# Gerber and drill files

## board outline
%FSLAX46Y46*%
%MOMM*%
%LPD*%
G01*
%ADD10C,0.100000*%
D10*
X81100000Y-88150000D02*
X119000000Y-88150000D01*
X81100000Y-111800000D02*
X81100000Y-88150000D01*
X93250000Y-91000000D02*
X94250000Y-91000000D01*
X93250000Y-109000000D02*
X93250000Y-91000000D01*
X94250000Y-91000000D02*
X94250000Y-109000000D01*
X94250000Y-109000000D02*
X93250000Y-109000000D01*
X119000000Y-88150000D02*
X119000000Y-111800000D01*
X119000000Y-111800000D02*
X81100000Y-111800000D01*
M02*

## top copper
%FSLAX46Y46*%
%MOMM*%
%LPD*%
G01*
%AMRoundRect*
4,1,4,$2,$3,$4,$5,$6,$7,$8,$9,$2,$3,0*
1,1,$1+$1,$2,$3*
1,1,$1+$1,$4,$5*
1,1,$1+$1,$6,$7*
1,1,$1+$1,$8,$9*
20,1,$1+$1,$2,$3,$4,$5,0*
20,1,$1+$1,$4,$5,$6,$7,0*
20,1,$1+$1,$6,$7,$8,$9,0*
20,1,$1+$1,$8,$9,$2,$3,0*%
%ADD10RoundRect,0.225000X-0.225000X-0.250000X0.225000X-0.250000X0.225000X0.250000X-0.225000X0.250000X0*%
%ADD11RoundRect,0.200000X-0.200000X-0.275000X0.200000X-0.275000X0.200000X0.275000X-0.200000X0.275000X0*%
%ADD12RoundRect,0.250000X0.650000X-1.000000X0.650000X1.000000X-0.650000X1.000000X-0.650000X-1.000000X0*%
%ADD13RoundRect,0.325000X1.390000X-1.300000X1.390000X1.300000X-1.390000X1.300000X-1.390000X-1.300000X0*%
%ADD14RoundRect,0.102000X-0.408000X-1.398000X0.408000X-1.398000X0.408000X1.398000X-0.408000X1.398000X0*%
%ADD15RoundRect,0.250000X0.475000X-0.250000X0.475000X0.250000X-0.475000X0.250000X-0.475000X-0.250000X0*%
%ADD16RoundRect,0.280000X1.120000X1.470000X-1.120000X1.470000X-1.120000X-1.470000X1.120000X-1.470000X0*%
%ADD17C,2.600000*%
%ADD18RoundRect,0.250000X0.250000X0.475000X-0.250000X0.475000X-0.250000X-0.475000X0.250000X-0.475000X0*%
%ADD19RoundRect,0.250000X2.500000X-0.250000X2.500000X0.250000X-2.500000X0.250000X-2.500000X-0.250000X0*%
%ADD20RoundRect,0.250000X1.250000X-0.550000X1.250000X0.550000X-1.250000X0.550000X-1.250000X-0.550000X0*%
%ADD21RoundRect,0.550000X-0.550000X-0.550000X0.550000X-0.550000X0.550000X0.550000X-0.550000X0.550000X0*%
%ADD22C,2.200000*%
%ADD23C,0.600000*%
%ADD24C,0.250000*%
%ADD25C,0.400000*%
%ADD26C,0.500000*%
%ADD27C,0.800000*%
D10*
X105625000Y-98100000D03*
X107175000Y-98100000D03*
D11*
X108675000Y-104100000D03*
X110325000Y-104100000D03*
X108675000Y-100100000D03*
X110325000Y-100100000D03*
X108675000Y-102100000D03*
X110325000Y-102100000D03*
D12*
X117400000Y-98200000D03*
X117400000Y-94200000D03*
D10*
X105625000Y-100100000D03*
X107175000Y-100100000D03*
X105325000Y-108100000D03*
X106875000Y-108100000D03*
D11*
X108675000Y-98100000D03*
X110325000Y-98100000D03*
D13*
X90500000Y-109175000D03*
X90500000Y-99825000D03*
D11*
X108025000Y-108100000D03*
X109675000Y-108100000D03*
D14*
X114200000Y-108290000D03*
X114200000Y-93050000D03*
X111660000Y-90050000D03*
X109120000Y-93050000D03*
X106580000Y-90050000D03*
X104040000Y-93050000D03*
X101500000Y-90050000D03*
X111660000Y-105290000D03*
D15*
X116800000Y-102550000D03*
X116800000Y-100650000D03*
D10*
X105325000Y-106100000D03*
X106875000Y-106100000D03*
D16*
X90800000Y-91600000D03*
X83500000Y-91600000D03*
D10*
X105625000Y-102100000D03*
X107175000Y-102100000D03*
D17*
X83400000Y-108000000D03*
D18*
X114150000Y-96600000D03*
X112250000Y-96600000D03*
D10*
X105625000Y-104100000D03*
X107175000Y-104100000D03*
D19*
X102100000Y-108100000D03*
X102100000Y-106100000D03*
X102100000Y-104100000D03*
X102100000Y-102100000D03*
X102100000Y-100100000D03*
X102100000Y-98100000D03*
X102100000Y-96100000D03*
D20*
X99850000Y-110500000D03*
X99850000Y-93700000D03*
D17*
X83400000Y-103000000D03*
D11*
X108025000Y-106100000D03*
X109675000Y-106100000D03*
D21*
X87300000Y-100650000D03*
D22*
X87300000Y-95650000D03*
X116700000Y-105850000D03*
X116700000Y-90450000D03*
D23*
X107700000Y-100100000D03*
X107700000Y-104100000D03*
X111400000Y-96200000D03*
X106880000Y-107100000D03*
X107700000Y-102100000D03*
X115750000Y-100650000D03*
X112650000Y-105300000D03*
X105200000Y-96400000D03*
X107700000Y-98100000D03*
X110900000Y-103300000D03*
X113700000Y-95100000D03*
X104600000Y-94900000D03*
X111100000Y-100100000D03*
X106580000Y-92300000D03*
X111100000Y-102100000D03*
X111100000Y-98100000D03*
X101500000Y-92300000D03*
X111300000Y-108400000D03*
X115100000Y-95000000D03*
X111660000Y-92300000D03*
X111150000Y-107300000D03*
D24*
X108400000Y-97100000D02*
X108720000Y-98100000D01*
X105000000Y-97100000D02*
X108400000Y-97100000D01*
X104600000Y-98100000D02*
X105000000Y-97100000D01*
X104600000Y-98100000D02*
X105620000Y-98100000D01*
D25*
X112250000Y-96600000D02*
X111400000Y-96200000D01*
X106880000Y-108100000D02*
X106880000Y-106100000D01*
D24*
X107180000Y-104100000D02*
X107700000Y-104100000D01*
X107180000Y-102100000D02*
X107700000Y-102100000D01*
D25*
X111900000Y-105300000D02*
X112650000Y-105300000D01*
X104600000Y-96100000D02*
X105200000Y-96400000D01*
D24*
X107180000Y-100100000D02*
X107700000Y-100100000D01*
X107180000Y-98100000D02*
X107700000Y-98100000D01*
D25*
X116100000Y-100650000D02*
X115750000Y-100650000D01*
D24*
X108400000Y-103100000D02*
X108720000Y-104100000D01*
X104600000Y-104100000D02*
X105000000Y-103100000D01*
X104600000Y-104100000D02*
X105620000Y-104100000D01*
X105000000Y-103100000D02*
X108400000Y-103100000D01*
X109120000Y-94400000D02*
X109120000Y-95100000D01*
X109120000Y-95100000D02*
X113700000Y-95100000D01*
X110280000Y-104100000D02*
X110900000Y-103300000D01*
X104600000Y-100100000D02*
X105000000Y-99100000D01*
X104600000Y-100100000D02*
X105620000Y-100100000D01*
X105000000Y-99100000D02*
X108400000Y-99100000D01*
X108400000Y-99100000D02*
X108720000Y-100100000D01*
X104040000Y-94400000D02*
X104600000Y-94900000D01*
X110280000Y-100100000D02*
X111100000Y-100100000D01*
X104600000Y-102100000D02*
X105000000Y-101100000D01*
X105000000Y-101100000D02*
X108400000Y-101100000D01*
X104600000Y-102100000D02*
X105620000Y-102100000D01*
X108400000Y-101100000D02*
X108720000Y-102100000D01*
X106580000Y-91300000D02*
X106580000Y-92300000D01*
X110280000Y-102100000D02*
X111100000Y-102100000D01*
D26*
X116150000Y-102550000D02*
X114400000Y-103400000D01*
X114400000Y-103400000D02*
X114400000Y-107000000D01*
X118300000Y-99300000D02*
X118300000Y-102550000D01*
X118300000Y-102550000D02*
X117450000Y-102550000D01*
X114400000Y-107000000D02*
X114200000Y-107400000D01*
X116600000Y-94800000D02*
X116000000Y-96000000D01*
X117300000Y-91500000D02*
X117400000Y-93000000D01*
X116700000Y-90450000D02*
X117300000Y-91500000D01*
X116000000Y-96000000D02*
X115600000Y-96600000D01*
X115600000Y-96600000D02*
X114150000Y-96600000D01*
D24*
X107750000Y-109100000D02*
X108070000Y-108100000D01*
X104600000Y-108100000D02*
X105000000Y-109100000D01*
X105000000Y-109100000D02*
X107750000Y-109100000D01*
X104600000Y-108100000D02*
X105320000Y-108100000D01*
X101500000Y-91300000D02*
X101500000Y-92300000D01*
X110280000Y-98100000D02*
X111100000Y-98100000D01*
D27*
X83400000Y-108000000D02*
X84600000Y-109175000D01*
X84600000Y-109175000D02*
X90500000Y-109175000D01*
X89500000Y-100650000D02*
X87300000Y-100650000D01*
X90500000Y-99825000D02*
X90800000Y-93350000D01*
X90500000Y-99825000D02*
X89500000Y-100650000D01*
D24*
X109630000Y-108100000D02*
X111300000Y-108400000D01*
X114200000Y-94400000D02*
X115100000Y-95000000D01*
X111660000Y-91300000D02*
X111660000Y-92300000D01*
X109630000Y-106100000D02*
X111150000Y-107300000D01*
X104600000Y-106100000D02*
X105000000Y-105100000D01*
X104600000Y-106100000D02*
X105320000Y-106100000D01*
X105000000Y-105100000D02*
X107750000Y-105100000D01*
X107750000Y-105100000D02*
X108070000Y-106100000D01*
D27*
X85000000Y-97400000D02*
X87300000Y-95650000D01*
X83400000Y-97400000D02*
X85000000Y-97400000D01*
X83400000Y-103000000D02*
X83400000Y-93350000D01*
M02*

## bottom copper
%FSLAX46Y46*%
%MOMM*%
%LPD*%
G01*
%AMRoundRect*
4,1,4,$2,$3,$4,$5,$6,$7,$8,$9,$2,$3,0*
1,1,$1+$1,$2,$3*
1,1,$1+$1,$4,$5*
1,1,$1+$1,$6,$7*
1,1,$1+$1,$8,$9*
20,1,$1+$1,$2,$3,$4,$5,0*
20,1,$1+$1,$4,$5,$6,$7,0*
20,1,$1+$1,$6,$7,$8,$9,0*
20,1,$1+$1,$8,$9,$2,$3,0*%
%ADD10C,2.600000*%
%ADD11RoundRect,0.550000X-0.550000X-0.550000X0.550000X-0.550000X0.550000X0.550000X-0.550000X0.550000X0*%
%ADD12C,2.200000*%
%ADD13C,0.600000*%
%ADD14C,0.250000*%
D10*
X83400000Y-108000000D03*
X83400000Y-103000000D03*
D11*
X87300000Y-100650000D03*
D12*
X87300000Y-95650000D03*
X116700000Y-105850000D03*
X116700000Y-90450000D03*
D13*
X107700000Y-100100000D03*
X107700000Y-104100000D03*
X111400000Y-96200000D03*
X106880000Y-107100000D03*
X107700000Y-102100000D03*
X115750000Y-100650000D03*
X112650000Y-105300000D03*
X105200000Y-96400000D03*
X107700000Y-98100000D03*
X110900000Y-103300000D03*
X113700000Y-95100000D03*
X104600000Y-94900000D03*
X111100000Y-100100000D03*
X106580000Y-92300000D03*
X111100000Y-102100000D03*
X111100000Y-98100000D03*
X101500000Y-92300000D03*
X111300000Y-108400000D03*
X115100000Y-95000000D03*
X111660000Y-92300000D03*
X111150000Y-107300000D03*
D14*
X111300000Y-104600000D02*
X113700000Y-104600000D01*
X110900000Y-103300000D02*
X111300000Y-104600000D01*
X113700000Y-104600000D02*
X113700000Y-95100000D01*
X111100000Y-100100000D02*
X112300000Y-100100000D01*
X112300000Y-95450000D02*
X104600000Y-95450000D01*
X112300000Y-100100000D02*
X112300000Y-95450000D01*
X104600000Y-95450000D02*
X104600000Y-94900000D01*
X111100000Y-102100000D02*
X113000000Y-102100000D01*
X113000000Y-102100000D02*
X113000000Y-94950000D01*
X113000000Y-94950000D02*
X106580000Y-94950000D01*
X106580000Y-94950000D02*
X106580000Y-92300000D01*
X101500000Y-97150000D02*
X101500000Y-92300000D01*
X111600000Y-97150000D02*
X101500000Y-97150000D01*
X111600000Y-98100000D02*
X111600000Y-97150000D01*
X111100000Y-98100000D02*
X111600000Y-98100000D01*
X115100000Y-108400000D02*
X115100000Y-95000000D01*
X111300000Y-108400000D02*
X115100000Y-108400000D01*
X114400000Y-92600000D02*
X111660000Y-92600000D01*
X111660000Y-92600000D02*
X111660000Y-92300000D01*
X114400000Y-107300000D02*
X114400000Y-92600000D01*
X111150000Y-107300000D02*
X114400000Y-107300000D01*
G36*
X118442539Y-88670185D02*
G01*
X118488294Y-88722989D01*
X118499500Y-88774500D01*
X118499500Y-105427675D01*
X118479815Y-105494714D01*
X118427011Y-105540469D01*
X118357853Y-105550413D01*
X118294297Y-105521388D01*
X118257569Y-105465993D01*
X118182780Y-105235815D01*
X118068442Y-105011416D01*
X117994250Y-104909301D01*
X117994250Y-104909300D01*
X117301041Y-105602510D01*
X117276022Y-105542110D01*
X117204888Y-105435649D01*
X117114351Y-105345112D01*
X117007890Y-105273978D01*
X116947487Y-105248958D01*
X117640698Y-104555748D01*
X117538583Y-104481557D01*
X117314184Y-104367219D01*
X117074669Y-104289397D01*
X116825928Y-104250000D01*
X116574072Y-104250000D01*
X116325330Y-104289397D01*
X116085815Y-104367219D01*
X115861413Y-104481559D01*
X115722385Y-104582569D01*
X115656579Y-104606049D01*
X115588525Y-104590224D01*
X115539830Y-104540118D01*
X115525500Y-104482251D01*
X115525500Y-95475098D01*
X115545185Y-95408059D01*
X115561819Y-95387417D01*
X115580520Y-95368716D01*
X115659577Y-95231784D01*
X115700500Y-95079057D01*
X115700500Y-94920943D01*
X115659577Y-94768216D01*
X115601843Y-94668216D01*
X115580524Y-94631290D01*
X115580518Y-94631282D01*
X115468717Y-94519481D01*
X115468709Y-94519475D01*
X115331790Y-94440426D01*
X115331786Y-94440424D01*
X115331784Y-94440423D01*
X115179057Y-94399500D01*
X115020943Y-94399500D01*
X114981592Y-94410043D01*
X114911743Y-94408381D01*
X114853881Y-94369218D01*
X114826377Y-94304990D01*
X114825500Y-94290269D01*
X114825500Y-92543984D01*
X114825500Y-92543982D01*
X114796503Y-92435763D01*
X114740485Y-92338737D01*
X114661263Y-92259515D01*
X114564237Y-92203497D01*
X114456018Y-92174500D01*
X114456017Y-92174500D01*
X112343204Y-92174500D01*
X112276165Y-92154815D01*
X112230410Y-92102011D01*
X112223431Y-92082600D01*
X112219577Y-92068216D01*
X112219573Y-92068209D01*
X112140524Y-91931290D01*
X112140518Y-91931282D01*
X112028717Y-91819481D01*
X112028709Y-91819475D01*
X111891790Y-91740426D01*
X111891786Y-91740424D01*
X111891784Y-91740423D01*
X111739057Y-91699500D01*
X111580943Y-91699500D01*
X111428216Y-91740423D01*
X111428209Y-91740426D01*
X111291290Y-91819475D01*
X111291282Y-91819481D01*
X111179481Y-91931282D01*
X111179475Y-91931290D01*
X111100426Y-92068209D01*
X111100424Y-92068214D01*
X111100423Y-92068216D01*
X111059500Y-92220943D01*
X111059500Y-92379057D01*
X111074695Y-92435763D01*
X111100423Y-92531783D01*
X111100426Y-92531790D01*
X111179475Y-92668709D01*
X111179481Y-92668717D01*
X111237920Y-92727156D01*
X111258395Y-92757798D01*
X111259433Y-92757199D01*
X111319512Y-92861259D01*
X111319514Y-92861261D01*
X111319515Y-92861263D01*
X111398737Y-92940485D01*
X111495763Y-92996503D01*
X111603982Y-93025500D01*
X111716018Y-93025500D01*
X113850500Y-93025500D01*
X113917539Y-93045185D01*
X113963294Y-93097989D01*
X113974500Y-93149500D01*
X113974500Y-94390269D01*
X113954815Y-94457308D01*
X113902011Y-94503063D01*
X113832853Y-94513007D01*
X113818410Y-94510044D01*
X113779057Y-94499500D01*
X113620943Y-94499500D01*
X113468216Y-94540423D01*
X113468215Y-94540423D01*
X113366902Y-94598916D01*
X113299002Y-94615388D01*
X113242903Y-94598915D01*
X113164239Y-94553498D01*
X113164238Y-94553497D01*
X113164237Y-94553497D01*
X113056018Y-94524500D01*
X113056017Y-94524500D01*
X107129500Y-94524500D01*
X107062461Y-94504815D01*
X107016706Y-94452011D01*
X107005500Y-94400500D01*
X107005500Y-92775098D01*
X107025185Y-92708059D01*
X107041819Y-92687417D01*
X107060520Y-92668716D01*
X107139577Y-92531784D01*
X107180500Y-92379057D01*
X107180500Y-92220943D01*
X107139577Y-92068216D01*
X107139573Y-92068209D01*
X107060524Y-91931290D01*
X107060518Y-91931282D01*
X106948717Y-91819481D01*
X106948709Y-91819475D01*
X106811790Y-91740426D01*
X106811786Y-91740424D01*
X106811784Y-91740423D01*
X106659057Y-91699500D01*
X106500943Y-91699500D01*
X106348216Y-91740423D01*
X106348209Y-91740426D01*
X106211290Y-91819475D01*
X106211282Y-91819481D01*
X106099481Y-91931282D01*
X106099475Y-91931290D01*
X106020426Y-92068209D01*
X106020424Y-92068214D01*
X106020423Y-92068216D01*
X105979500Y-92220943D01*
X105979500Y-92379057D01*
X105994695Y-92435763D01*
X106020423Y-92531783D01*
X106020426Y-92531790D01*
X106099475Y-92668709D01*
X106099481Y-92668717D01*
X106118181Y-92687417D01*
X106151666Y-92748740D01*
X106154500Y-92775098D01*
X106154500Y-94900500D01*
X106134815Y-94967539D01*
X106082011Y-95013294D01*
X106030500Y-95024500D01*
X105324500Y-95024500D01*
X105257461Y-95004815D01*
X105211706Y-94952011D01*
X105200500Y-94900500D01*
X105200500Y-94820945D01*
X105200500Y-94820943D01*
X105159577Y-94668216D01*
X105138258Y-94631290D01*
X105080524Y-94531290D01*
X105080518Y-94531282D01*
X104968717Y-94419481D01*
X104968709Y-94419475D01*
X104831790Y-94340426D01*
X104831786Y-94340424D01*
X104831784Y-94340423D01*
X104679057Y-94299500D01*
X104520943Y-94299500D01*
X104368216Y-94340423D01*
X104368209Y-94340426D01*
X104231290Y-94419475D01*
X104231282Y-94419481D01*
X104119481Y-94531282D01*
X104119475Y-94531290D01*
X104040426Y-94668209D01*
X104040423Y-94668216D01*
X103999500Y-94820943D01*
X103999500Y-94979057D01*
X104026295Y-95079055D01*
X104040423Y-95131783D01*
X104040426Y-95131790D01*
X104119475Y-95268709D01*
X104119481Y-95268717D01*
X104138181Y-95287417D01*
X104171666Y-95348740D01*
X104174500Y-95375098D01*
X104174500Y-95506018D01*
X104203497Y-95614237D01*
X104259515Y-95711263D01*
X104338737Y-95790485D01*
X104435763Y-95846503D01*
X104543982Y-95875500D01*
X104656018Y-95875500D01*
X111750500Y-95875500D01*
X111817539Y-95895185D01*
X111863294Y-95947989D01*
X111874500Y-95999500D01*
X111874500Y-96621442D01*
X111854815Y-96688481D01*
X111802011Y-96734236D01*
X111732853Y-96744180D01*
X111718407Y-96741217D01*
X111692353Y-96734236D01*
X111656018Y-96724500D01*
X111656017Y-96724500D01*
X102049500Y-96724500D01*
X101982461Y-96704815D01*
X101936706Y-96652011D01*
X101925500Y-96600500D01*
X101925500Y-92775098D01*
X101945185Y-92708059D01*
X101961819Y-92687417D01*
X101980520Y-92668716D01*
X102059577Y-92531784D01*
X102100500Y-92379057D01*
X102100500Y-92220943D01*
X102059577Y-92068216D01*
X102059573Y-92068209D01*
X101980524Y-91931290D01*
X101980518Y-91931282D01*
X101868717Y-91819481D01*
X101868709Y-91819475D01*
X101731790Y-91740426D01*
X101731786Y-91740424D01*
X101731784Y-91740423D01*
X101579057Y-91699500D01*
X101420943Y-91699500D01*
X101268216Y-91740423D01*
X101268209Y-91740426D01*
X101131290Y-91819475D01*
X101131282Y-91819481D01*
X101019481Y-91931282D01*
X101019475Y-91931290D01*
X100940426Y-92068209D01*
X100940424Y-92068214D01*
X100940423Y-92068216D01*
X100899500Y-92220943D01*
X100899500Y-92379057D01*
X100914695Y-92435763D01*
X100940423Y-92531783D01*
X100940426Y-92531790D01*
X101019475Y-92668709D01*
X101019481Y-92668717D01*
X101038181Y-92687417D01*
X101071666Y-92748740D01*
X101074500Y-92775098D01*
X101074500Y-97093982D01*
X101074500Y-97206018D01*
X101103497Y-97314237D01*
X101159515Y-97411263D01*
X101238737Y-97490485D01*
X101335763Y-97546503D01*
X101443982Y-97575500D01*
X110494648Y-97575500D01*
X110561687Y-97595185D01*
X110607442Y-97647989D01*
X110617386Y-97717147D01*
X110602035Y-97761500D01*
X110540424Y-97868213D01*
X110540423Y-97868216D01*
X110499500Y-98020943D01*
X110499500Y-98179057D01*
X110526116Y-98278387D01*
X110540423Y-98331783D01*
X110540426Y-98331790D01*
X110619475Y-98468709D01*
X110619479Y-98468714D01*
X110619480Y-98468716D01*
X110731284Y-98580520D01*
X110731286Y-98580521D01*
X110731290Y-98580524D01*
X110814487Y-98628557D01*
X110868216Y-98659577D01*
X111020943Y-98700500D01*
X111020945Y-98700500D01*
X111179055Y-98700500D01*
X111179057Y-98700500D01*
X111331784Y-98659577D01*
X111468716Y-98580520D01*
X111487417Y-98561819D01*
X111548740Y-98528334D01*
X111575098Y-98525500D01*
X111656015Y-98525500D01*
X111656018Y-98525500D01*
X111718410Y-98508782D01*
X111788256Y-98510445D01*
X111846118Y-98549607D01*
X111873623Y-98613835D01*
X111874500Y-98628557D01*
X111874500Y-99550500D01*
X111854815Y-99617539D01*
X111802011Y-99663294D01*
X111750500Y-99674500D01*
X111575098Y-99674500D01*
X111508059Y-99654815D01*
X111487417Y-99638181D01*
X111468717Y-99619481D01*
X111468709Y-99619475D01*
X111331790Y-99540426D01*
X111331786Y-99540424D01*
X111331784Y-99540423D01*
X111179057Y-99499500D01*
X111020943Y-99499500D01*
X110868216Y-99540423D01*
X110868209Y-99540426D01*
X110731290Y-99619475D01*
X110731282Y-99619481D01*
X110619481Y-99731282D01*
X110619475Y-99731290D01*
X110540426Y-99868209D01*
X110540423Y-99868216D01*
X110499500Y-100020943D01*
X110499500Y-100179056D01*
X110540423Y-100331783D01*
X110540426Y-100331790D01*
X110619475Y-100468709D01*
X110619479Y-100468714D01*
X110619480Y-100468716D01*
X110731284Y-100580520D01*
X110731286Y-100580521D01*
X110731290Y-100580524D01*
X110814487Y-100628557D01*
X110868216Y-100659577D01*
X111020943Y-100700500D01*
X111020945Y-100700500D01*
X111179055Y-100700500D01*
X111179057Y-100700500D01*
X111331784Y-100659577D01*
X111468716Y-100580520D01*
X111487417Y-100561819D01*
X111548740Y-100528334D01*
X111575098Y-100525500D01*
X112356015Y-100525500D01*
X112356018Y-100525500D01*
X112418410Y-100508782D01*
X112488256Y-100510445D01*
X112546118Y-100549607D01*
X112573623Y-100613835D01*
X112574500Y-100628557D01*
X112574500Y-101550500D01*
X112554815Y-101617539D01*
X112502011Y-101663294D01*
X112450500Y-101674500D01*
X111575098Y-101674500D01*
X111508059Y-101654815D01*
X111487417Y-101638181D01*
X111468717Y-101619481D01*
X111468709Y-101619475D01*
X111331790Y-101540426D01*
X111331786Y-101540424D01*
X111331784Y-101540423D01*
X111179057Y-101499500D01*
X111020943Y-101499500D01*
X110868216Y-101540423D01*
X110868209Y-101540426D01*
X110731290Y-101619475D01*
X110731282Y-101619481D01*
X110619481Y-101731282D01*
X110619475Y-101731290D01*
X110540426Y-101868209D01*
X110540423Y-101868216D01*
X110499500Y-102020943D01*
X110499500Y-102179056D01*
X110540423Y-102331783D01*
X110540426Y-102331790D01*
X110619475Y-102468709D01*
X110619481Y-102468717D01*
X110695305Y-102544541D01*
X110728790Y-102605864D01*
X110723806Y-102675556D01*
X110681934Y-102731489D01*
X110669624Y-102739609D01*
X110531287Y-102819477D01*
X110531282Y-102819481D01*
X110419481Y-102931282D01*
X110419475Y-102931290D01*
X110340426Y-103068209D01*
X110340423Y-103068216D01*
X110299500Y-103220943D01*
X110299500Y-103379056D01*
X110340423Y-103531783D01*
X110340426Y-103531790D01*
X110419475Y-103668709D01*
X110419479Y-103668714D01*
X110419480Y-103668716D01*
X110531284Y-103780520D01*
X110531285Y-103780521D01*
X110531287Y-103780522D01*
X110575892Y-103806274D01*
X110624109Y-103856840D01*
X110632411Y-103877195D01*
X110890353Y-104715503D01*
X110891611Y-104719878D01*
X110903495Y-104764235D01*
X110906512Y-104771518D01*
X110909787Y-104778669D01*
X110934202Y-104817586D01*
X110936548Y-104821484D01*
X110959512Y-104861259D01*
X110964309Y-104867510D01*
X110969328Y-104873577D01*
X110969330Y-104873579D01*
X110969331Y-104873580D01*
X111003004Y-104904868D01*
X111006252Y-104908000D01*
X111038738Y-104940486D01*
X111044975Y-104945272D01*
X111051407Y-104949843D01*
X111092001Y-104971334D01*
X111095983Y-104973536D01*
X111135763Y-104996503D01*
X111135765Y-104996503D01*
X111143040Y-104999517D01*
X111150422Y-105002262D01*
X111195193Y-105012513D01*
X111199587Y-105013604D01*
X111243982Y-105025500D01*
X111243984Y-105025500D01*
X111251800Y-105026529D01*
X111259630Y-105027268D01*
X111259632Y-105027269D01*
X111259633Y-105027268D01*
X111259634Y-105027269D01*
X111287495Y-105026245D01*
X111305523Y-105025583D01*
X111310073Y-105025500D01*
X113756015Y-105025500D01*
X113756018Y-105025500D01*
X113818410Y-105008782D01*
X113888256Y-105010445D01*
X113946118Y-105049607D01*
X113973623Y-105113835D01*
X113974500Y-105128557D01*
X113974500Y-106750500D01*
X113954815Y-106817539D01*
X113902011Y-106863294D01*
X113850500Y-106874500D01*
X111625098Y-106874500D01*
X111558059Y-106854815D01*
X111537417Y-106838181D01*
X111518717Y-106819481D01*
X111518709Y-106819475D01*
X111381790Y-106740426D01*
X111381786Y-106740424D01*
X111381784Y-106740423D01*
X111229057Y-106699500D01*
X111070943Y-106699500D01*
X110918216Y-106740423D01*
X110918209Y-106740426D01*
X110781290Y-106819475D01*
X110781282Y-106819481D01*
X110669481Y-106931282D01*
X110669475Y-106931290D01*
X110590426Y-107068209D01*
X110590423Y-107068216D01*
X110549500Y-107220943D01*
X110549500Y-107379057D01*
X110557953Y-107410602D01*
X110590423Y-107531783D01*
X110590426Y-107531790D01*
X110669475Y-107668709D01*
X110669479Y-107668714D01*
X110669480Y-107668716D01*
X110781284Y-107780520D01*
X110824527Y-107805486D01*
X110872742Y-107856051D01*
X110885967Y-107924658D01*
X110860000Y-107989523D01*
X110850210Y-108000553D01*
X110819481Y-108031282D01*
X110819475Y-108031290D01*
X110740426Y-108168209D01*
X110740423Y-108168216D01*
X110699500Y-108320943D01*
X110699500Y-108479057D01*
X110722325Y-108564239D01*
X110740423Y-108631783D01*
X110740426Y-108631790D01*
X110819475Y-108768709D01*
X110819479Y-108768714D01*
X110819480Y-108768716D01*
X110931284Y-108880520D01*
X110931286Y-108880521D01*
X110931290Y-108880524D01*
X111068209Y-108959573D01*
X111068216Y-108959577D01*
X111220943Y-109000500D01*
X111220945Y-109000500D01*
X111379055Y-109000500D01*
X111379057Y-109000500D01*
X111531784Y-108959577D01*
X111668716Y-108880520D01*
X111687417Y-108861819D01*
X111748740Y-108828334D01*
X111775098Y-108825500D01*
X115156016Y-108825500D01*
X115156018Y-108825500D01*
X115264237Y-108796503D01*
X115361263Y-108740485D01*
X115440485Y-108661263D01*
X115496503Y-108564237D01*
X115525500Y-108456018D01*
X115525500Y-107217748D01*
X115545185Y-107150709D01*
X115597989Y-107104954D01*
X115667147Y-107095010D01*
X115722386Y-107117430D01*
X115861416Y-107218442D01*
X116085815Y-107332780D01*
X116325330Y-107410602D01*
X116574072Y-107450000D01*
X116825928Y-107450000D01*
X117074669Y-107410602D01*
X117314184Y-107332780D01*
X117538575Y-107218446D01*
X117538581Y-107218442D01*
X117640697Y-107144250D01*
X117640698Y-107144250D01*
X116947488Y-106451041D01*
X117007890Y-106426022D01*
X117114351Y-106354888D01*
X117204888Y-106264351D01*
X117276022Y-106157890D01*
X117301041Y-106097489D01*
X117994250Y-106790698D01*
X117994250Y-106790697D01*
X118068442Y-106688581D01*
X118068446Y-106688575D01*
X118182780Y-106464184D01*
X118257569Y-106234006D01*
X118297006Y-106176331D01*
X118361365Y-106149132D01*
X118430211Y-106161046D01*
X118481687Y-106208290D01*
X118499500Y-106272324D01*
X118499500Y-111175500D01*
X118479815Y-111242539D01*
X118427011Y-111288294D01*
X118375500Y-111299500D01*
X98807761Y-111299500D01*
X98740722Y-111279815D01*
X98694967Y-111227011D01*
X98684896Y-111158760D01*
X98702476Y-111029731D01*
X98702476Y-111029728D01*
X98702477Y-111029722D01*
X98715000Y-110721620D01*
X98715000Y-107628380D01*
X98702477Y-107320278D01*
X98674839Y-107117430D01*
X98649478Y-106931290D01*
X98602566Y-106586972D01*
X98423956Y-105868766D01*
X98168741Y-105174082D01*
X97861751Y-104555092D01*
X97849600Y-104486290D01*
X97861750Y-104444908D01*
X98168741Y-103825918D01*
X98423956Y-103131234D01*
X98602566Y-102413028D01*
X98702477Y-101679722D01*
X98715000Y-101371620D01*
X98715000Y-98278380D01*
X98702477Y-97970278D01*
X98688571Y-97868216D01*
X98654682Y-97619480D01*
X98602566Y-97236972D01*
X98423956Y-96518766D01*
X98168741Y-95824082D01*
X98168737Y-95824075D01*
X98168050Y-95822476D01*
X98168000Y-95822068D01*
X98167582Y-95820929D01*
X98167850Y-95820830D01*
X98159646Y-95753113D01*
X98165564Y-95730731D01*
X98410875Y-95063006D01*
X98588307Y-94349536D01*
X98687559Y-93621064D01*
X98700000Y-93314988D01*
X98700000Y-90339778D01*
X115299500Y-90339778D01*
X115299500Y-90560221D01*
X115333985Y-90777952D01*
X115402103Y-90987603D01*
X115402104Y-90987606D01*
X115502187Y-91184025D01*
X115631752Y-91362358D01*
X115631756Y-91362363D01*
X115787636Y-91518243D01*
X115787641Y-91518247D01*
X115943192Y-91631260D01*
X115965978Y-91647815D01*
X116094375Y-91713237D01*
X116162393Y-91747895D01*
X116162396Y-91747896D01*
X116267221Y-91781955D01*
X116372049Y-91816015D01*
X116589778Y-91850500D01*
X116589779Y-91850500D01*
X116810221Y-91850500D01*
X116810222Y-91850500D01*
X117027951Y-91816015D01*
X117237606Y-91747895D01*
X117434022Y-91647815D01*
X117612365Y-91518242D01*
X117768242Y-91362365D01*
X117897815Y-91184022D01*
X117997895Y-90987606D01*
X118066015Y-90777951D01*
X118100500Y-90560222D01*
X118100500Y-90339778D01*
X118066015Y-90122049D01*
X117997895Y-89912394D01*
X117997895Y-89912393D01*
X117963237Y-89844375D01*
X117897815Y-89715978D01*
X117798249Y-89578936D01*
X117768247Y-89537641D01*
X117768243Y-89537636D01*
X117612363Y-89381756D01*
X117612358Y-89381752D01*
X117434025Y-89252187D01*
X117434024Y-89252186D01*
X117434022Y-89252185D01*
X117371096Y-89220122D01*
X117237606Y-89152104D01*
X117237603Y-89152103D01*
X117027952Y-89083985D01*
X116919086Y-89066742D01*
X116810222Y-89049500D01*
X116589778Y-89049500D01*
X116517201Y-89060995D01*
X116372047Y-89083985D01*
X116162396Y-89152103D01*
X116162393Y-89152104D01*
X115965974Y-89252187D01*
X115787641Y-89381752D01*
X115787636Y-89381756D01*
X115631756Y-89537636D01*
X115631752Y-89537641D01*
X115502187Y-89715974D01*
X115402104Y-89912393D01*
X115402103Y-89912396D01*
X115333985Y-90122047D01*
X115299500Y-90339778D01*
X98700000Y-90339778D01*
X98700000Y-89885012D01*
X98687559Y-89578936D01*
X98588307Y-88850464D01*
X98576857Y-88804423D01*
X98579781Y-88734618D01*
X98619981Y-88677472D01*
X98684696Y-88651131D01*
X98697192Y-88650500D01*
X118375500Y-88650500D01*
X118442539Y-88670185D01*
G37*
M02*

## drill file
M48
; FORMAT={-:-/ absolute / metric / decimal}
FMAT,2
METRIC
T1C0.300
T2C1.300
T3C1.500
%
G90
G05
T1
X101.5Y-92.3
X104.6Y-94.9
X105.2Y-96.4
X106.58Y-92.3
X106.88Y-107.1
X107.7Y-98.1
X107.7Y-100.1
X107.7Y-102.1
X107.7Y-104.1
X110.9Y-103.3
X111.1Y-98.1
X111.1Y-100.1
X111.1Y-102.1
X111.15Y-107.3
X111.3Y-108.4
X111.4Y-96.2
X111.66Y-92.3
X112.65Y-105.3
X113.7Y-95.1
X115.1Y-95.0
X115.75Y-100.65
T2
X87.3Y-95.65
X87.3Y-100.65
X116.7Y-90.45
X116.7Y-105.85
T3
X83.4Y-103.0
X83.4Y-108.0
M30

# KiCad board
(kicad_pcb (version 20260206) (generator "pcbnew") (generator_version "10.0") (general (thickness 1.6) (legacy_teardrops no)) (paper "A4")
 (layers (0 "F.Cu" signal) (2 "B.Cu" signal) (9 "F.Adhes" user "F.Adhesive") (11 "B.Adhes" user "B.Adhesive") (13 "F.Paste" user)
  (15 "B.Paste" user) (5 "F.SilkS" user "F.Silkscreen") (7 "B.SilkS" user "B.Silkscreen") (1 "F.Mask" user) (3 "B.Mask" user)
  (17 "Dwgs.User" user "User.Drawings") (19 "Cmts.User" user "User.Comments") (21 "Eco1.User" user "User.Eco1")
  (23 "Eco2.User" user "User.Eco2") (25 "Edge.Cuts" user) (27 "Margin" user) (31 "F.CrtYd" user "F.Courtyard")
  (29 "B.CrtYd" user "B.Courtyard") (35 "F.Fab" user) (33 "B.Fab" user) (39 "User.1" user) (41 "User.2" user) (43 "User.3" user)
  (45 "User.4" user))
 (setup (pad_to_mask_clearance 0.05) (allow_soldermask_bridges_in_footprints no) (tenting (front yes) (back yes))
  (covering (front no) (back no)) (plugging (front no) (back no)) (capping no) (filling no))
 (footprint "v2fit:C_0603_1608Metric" (layer "F.Cu") (at 106.4 98.1)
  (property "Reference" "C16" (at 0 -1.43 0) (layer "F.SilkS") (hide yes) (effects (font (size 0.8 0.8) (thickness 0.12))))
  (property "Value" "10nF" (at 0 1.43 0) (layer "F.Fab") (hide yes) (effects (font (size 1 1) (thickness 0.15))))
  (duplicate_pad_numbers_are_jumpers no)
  (pad "1" smd roundrect (at -0.775 0) (size 0.9 0.95) (layers "F.Cu" "F.Mask" "F.Paste") (roundrect_rratio 0.25) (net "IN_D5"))
  (pad "2" smd roundrect (at 0.775 0) (size 0.9 0.95) (layers "F.Cu" "F.Mask" "F.Paste") (roundrect_rratio 0.25) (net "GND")))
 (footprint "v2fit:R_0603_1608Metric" (layer "F.Cu") (at 109.5 104.1)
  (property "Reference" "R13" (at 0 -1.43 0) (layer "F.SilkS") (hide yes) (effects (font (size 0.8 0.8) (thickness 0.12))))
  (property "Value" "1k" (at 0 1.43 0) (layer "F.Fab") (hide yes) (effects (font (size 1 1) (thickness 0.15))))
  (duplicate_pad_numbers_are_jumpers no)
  (pad "1" smd roundrect (at -0.825 0) (size 0.8 0.95) (layers "F.Cu" "F.Mask" "F.Paste") (roundrect_rratio 0.25) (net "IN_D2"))
  (pad "2" smd roundrect (at 0.825 0) (size 0.8 0.95) (layers "F.Cu" "F.Mask" "F.Paste") (roundrect_rratio 0.25) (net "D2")))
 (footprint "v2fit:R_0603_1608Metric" (layer "F.Cu") (at 109.5 100.1)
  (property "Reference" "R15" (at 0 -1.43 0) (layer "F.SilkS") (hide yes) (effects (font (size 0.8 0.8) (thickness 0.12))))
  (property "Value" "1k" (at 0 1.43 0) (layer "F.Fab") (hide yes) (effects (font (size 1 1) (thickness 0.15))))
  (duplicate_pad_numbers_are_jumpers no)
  (pad "1" smd roundrect (at -0.825 0) (size 0.8 0.95) (layers "F.Cu" "F.Mask" "F.Paste") (roundrect_rratio 0.25) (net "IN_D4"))
  (pad "2" smd roundrect (at 0.825 0) (size 0.8 0.95) (layers "F.Cu" "F.Mask" "F.Paste") (roundrect_rratio 0.25) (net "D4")))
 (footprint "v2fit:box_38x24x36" (layer "F.Cu") (at 100 100)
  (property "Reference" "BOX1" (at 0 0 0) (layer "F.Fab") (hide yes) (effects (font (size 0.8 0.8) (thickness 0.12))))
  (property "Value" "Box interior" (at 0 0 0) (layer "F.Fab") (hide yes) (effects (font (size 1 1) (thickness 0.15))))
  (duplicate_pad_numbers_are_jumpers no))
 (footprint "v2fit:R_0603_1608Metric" (layer "F.Cu") (at 109.5 102.1)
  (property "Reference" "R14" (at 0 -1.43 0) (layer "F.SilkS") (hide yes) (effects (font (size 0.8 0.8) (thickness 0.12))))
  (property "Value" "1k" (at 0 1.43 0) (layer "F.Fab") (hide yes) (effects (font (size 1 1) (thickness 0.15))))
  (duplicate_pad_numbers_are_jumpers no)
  (pad "1" smd roundrect (at -0.825 0) (size 0.8 0.95) (layers "F.Cu" "F.Mask" "F.Paste") (roundrect_rratio 0.25) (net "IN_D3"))
  (pad "2" smd roundrect (at 0.825 0) (size 0.8 0.95) (layers "F.Cu" "F.Mask" "F.Paste") (roundrect_rratio 0.25) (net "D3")))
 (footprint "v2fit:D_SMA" (layer "F.Cu") (at 117.4 96.2 90)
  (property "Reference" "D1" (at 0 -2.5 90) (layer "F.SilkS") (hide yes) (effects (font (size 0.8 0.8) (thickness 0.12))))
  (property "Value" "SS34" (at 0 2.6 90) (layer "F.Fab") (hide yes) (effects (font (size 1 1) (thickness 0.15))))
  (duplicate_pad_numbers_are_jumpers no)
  (pad "1" smd roundrect (at -2 0 90) (size 2.5 1.8) (layers "F.Cu" "F.Mask" "F.Paste") (roundrect_rratio 0.1388888889) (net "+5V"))
  (pad "2" smd roundrect (at 2 0 90) (size 2.5 1.8) (layers "F.Cu" "F.Mask" "F.Paste") (roundrect_rratio 0.1388888889) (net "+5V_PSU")))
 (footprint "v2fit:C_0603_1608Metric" (layer "F.Cu") (at 106.4 100.1)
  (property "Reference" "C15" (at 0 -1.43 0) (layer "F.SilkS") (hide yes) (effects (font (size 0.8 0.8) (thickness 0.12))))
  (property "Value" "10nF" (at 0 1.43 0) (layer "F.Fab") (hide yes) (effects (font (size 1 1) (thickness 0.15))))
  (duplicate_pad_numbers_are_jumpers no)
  (pad "1" smd roundrect (at -0.775 0) (size 0.9 0.95) (layers "F.Cu" "F.Mask" "F.Paste") (roundrect_rratio 0.25) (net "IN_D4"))
  (pad "2" smd roundrect (at 0.775 0) (size 0.9 0.95) (layers "F.Cu" "F.Mask" "F.Paste") (roundrect_rratio 0.25) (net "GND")))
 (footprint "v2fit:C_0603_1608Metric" (layer "F.Cu") (at 106.1 108.1)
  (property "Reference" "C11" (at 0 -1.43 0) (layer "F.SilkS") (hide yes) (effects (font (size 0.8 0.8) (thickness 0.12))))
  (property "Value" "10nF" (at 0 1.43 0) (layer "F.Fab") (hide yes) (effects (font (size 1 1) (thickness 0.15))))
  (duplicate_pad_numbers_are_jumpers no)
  (pad "1" smd roundrect (at -0.775 0) (size 0.9 0.95) (layers "F.Cu" "F.Mask" "F.Paste") (roundrect_rratio 0.25) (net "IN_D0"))
  (pad "2" smd roundrect (at 0.775 0) (size 0.9 0.95) (layers "F.Cu" "F.Mask" "F.Paste") (roundrect_rratio 0.25) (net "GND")))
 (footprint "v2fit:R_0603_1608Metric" (layer "F.Cu") (at 109.5 98.1)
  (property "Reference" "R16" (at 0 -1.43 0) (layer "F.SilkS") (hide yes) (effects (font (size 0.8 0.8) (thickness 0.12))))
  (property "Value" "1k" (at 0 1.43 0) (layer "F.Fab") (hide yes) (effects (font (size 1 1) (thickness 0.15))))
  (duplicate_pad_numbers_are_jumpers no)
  (pad "1" smd roundrect (at -0.825 0) (size 0.8 0.95) (layers "F.Cu" "F.Mask" "F.Paste") (roundrect_rratio 0.25) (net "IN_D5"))
  (pad "2" smd roundrect (at 0.825 0) (size 0.8 0.95) (layers "F.Cu" "F.Mask" "F.Paste") (roundrect_rratio 0.25) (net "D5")))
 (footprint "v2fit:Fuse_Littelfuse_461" (layer "F.Cu") (at 90.5 104.5 90)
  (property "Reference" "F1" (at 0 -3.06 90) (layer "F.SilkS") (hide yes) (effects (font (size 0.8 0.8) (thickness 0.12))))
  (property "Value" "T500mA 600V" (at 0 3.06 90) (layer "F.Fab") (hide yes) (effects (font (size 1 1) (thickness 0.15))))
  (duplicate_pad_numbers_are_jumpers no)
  (pad "1" smd roundrect (at -4.675 0 90) (size 3.25 3.43) (layers "F.Cu" "F.Mask" "F.Paste") (roundrect_rratio 0.1) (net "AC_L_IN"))
  (pad "2" smd roundrect (at 4.675 0 90) (size 3.25 3.43) (layers "F.Cu" "F.Mask" "F.Paste") (roundrect_rratio 0.1) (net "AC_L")))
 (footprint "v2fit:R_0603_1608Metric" (layer "F.Cu") (at 108.85 108.1)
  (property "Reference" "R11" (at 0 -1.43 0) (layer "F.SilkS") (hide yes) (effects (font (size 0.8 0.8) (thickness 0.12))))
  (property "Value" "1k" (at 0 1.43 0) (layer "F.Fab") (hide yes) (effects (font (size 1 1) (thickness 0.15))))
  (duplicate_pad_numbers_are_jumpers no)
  (pad "1" smd roundrect (at -0.825 0) (size 0.8 0.95) (layers "F.Cu" "F.Mask" "F.Paste") (roundrect_rratio 0.25) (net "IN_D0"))
  (pad "2" smd roundrect (at 0.825 0) (size 0.8 0.95) (layers "F.Cu" "F.Mask" "F.Paste") (roundrect_rratio 0.25) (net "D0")))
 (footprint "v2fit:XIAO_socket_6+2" (layer "F.Cu") (at 106.58 99.17)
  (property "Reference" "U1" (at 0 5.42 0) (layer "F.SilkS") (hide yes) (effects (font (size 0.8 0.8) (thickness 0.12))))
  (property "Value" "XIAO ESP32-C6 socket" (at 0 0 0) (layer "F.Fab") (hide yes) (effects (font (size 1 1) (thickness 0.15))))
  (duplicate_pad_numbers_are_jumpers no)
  (pad "5V" smd roundrect (at 7.62 9.12) (size 1.02 3) (layers "F.Cu" "F.Mask" "F.Paste") (roundrect_rratio 0.1) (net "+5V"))
  (pad "D0" smd roundrect (at 7.62 -6.12) (size 1.02 3) (layers "F.Cu" "F.Mask" "F.Paste") (roundrect_rratio 0.1) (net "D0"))
  (pad "D1" smd roundrect (at 5.08 -9.12) (size 1.02 3) (layers "F.Cu" "F.Mask" "F.Paste") (roundrect_rratio 0.1) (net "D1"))
  (pad "D2" smd roundrect (at 2.54 -6.12) (size 1.02 3) (layers "F.Cu" "F.Mask" "F.Paste") (roundrect_rratio 0.1) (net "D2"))
  (pad "D3" smd roundrect (at 0 -9.12) (size 1.02 3) (layers "F.Cu" "F.Mask" "F.Paste") (roundrect_rratio 0.1) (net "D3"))
  (pad "D4" smd roundrect (at -2.54 -6.12) (size 1.02 3) (layers "F.Cu" "F.Mask" "F.Paste") (roundrect_rratio 0.1) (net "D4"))
  (pad "D5" smd roundrect (at -5.08 -9.12) (size 1.02 3) (layers "F.Cu" "F.Mask" "F.Paste") (roundrect_rratio 0.1) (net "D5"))
  (pad "GND" smd roundrect (at 5.08 6.12) (size 1.02 3) (layers "F.Cu" "F.Mask" "F.Paste") (roundrect_rratio 0.1) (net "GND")))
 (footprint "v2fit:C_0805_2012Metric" (layer "F.Cu") (at 116.8 101.6 90)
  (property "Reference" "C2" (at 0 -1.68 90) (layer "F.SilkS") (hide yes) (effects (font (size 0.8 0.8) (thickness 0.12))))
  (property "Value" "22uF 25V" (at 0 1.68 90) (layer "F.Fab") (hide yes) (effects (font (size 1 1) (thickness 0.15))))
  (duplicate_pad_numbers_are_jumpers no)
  (pad "1" smd roundrect (at -0.95 0 90) (size 1 1.45) (layers "F.Cu" "F.Mask" "F.Paste") (roundrect_rratio 0.25) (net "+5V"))
  (pad "2" smd roundrect (at 0.95 0 90) (size 1 1.45) (layers "F.Cu" "F.Mask" "F.Paste") (roundrect_rratio 0.25) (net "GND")))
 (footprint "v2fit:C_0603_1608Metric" (layer "F.Cu") (at 106.1 106.1)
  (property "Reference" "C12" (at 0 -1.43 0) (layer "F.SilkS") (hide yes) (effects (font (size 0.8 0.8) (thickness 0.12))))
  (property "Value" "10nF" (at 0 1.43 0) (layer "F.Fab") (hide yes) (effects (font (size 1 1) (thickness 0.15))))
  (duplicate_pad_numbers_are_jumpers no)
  (pad "1" smd roundrect (at -0.775 0) (size 0.9 0.95) (layers "F.Cu" "F.Mask" "F.Paste") (roundrect_rratio 0.25) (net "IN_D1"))
  (pad "2" smd roundrect (at 0.775 0) (size 0.9 0.95) (layers "F.Cu" "F.Mask" "F.Paste") (roundrect_rratio 0.25) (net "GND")))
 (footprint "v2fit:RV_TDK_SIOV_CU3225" (layer "F.Cu") (at 87.15 91.6 180)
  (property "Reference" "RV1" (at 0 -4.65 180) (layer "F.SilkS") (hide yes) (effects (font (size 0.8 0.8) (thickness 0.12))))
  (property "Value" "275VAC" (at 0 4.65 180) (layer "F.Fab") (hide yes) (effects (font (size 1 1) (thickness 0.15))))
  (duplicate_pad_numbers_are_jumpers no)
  (pad "1" smd roundrect (at -3.65 0 180) (size 2.8 3.5) (layers "F.Cu" "F.Mask" "F.Paste") (roundrect_rratio 0.1) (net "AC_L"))
  (pad "2" smd roundrect (at 3.65 0 180) (size 2.8 3.5) (layers "F.Cu" "F.Mask" "F.Paste") (roundrect_rratio 0.1) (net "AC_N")))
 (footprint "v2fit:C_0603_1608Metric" (layer "F.Cu") (at 106.4 102.1)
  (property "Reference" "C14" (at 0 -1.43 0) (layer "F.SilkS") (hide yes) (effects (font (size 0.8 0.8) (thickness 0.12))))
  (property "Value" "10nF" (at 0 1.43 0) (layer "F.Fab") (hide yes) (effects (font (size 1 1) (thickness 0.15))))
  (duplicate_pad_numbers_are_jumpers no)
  (pad "1" smd roundrect (at -0.775 0) (size 0.9 0.95) (layers "F.Cu" "F.Mask" "F.Paste") (roundrect_rratio 0.25) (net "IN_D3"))
  (pad "2" smd roundrect (at 0.775 0) (size 0.9 0.95) (layers "F.Cu" "F.Mask" "F.Paste") (roundrect_rratio 0.25) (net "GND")))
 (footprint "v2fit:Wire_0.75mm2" (layer "F.Cu") (at 83.4 108)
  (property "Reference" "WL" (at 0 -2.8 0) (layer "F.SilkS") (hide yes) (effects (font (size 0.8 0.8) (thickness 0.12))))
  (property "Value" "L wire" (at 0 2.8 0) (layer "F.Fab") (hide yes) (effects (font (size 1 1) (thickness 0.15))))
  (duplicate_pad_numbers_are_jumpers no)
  (pad "1" thru_hole circle (at 0 0) (size 2.6 2.6) (drill 1.5) (layers "*.Cu" "*.Mask") (remove_unused_layers no) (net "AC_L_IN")))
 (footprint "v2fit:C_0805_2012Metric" (layer "F.Cu") (at 113.2 96.6 180)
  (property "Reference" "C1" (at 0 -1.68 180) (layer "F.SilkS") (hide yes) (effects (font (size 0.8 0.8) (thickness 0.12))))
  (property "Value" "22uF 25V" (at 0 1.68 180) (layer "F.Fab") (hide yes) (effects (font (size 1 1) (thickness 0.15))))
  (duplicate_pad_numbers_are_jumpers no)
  (pad "1" smd roundrect (at -0.95 0 180) (size 1 1.45) (layers "F.Cu" "F.Mask" "F.Paste") (roundrect_rratio 0.25) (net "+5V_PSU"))
  (pad "2" smd roundrect (at 0.95 0 180) (size 1 1.45) (layers "F.Cu" "F.Mask" "F.Paste") (roundrect_rratio 0.25) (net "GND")))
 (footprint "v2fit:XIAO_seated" (layer "F.Cu") (at 106.58 99.17)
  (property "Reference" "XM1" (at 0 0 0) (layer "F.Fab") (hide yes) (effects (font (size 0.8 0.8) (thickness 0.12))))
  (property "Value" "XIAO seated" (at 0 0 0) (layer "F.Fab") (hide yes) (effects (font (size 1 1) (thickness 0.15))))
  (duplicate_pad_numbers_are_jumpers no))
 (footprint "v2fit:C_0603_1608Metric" (layer "F.Cu") (at 106.4 104.1)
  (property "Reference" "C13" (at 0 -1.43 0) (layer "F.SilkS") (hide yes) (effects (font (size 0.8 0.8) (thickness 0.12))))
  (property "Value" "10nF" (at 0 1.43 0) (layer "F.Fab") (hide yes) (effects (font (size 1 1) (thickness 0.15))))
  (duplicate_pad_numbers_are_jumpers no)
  (pad "1" smd roundrect (at -0.775 0) (size 0.9 0.95) (layers "F.Cu" "F.Mask" "F.Paste") (roundrect_rratio 0.25) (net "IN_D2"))
  (pad "2" smd roundrect (at 0.775 0) (size 0.9 0.95) (layers "F.Cu" "F.Mask" "F.Paste") (roundrect_rratio 0.25) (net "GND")))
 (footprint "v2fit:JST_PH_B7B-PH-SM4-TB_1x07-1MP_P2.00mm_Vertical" (layer "F.Cu") (at 101.6 102.1 90)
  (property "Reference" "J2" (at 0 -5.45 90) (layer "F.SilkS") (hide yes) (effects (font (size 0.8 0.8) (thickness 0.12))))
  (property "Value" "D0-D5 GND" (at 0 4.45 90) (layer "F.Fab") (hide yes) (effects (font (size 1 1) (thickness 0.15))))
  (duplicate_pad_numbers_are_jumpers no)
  (pad "1" smd roundrect (at -6 0.5 90) (size 1 5.5) (layers "F.Cu" "F.Mask" "F.Paste") (roundrect_rratio 0.25) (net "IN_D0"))
  (pad "2" smd roundrect (at -4 0.5 90) (size 1 5.5) (layers "F.Cu" "F.Mask" "F.Paste") (roundrect_rratio 0.25) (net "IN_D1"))
  (pad "3" smd roundrect (at -2 0.5 90) (size 1 5.5) (layers "F.Cu" "F.Mask" "F.Paste") (roundrect_rratio 0.25) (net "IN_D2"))
  (pad "4" smd roundrect (at 0 0.5 90) (size 1 5.5) (layers "F.Cu" "F.Mask" "F.Paste") (roundrect_rratio 0.25) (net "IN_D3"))
  (pad "5" smd roundrect (at 2 0.5 90) (size 1 5.5) (layers "F.Cu" "F.Mask" "F.Paste") (roundrect_rratio 0.25) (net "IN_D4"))
  (pad "6" smd roundrect (at 4 0.5 90) (size 1 5.5) (layers "F.Cu" "F.Mask" "F.Paste") (roundrect_rratio 0.25) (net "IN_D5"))
  (pad "7" smd roundrect (at 6 0.5 90) (size 1 5.5) (layers "F.Cu" "F.Mask" "F.Paste") (roundrect_rratio 0.25) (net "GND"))
  (pad "MP" smd roundrect (at -8.4 -1.75 90) (size 1.6 3) (layers "F.Cu" "F.Mask" "F.Paste") (roundrect_rratio 0.15625))
  (pad "MP" smd roundrect (at 8.4 -1.75 90) (size 1.6 3) (layers "F.Cu" "F.Mask" "F.Paste") (roundrect_rratio 0.15625)))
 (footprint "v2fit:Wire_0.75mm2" (layer "F.Cu") (at 83.4 103)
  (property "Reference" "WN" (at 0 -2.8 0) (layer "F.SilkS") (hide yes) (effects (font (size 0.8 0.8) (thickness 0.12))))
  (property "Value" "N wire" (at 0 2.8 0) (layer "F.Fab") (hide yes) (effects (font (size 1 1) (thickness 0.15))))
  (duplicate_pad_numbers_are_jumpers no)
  (pad "1" thru_hole circle (at 0 0) (size 2.6 2.6) (drill 1.5) (layers "*.Cu" "*.Mask") (remove_unused_layers no) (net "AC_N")))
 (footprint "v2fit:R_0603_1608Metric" (layer "F.Cu") (at 108.85 106.1)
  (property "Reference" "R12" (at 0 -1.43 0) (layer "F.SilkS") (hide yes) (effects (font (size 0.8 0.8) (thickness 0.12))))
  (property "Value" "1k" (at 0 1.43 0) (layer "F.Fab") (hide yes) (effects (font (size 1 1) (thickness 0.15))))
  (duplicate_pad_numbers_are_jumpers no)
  (pad "1" smd roundrect (at -0.825 0) (size 0.8 0.95) (layers "F.Cu" "F.Mask" "F.Paste") (roundrect_rratio 0.25) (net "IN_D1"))
  (pad "2" smd roundrect (at 0.825 0) (size 0.8 0.95) (layers "F.Cu" "F.Mask" "F.Paste") (roundrect_rratio 0.25) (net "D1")))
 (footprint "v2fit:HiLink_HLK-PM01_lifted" (layer "B.Cu") (at 87.3 100.65)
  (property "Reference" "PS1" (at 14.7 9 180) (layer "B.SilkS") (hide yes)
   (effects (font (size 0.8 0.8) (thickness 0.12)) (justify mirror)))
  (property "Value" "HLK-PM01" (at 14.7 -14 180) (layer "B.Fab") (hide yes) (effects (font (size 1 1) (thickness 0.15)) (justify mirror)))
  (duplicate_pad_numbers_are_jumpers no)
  (pad "1" thru_hole roundrect (at 0 0) (size 2.2 2.2) (drill 1.3) (layers "*.Cu" "*.Mask") (remove_unused_layers no)
   (roundrect_rratio 0.25) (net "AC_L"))
  (pad "2" thru_hole circle (at 0 -5) (size 2.2 2.2) (drill 1.3) (layers "*.Cu" "*.Mask") (remove_unused_layers no) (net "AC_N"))
  (pad "3" thru_hole circle (at 29.4 5.2) (size 2.2 2.2) (drill 1.3) (layers "*.Cu" "*.Mask") (remove_unused_layers no) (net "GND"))
  (pad "4" thru_hole circle (at 29.4 -10.2) (size 2.2 2.2) (drill 1.3) (layers "*.Cu" "*.Mask") (remove_unused_layers no) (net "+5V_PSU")))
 (gr_line (start 81.1 88.15) (end 119 88.15) (stroke (width 0.1) (type default)) (layer "Edge.Cuts"))
 (gr_line (start 81.1 111.8) (end 81.1 88.15) (stroke (width 0.1) (type default)) (layer "Edge.Cuts"))
 (gr_line (start 93.25 91) (end 94.25 91) (stroke (width 0.1) (type default)) (layer "Edge.Cuts"))
 (gr_line (start 93.25 109) (end 93.25 91) (stroke (width 0.1) (type default)) (layer "Edge.Cuts"))
 (gr_line (start 94.25 91) (end 94.25 109) (stroke (width 0.1) (type default)) (layer "Edge.Cuts"))
 (gr_line (start 94.25 109) (end 93.25 109) (stroke (width 0.1) (type default)) (layer "Edge.Cuts"))
 (gr_line (start 119 88.15) (end 119 111.8) (stroke (width 0.1) (type default)) (layer "Edge.Cuts"))
 (gr_line (start 119 111.8) (end 81.1 111.8) (stroke (width 0.1) (type default)) (layer "Edge.Cuts"))
 (segment (start 108.4 97.1) (end 108.72 98.1) (width 0.25) (layer "F.Cu") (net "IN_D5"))
 (segment (start 105 97.1) (end 108.4 97.1) (width 0.25) (layer "F.Cu") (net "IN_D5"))
 (segment (start 104.6 98.1) (end 105 97.1) (width 0.25) (layer "F.Cu") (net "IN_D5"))
 (segment (start 104.6 98.1) (end 105.62 98.1) (width 0.25) (layer "F.Cu") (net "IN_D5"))
 (segment (start 112.25 96.6) (end 111.4 96.2) (width 0.4) (layer "F.Cu") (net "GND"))
 (segment (start 106.88 108.1) (end 106.88 106.1) (width 0.4) (layer "F.Cu") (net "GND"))
 (segment (start 107.18 104.1) (end 107.7 104.1) (width 0.25) (layer "F.Cu") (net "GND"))
 (segment (start 107.18 102.1) (end 107.7 102.1) (width 0.25) (layer "F.Cu") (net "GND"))
 (segment (start 111.9 105.3) (end 112.65 105.3) (width 0.4) (layer "F.Cu") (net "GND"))
 (segment (start 104.6 96.1) (end 105.2 96.4) (width 0.4) (layer "F.Cu") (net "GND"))
 (segment (start 107.18 100.1) (end 107.7 100.1) (width 0.25) (layer "F.Cu") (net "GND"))
 (segment (start 107.18 98.1) (end 107.7 98.1) (width 0.25) (layer "F.Cu") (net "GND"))
 (segment (start 116.1 100.65) (end 115.75 100.65) (width 0.4) (layer "F.Cu") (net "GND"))
 (via (at 107.7 100.1) (size 0.6) (drill 0.3) (layers "F.Cu" "B.Cu") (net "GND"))
 (via (at 107.7 104.1) (size 0.6) (drill 0.3) (layers "F.Cu" "B.Cu") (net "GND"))
 (via (at 111.4 96.2) (size 0.6) (drill 0.3) (layers "F.Cu" "B.Cu") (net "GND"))
 (via (at 106.88 107.1) (size 0.6) (drill 0.3) (layers "F.Cu" "B.Cu") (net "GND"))
 (via (at 107.7 102.1) (size 0.6) (drill 0.3) (layers "F.Cu" "B.Cu") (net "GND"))
 (via (at 115.75 100.65) (size 0.6) (drill 0.3) (layers "F.Cu" "B.Cu") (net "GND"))
 (via (at 112.65 105.3) (size 0.6) (drill 0.3) (layers "F.Cu" "B.Cu") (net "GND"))
 (via (at 105.2 96.4) (size 0.6) (drill 0.3) (layers "F.Cu" "B.Cu") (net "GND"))
 (via (at 107.7 98.1) (size 0.6) (drill 0.3) (layers "F.Cu" "B.Cu") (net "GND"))
 (segment (start 108.4 103.1) (end 108.72 104.1) (width 0.25) (layer "F.Cu") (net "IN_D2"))
 (segment (start 104.6 104.1) (end 105 103.1) (width 0.25) (layer "F.Cu") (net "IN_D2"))
 (segment (start 104.6 104.1) (end 105.62 104.1) (width 0.25) (layer "F.Cu") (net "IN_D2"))
 (segment (start 105 103.1) (end 108.4 103.1) (width 0.25) (layer "F.Cu") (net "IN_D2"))
 (segment (start 109.12 94.4) (end 109.12 95.1) (width 0.25) (layer "F.Cu") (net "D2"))
 (segment (start 109.12 95.1) (end 113.7 95.1) (width 0.25) (layer "F.Cu") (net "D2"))
 (segment (start 110.28 104.1) (end 110.9 103.3) (width 0.25) (layer "F.Cu") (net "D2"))
 (via (at 110.9 103.3) (size 0.6) (drill 0.3) (layers "F.Cu" "B.Cu") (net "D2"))
 (via (at 113.7 95.1) (size 0.6) (drill 0.3) (layers "F.Cu" "B.Cu") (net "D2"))
 (segment (start 111.3 104.6) (end 113.7 104.6) (width 0.25) (layer "B.Cu") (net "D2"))
 (segment (start 110.9 103.3) (end 111.3 104.6) (width 0.25) (layer "B.Cu") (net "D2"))
 (segment (start 113.7 104.6) (end 113.7 95.1) (width 0.25) (layer "B.Cu") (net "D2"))
 (segment (start 104.6 100.1) (end 105 99.1) (width 0.25) (layer "F.Cu") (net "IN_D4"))
 (segment (start 104.6 100.1) (end 105.62 100.1) (width 0.25) (layer "F.Cu") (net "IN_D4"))
 (segment (start 105 99.1) (end 108.4 99.1) (width 0.25) (layer "F.Cu") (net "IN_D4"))
 (segment (start 108.4 99.1) (end 108.72 100.1) (width 0.25) (layer "F.Cu") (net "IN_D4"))
 (segment (start 104.04 94.4) (end 104.6 94.9) (width 0.25) (layer "F.Cu") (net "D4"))
 (segment (start 110.28 100.1) (end 111.1 100.1) (width 0.25) (layer "F.Cu") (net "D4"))
 (via (at 104.6 94.9) (size 0.6) (drill 0.3) (layers "F.Cu" "B.Cu") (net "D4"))
 (via (at 111.1 100.1) (size 0.6) (drill 0.3) (layers "F.Cu" "B.Cu") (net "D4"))
 (segment (start 111.1 100.1) (end 112.3 100.1) (width 0.25) (layer "B.Cu") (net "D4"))
 (segment (start 112.3 95.45) (end 104.6 95.45) (width 0.25) (layer "B.Cu") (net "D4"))
 (segment (start 112.3 100.1) (end 112.3 95.45) (width 0.25) (layer "B.Cu") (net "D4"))
 (segment (start 104.6 95.45) (end 104.6 94.9) (width 0.25) (layer "B.Cu") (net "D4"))
 (segment (start 104.6 102.1) (end 105 101.1) (width 0.25) (layer "F.Cu") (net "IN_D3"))
 (segment (start 105 101.1) (end 108.4 101.1) (width 0.25) (layer "F.Cu") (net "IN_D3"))
 (segment (start 104.6 102.1) (end 105.62 102.1) (width 0.25) (layer "F.Cu") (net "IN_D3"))
 (segment (start 108.4 101.1) (end 108.72 102.1) (width 0.25) (layer "F.Cu") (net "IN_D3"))
 (segment (start 106.58 91.3) (end 106.58 92.3) (width 0.25) (layer "F.Cu") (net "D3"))
 (segment (start 110.28 102.1) (end 111.1 102.1) (width 0.25) (layer "F.Cu") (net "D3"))
 (via (at 106.58 92.3) (size 0.6) (drill 0.3) (layers "F.Cu" "B.Cu") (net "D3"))
 (via (at 111.1 102.1) (size 0.6) (drill 0.3) (layers "F.Cu" "B.Cu") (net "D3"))
 (segment (start 111.1 102.1) (end 113 102.1) (width 0.25) (layer "B.Cu") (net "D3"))
 (segment (start 113 102.1) (end 113 94.95) (width 0.25) (layer "B.Cu") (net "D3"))
 (segment (start 113 94.95) (end 106.58 94.95) (width 0.25) (layer "B.Cu") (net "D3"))
 (segment (start 106.58 94.95) (end 106.58 92.3) (width 0.25) (layer "B.Cu") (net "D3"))
 (segment (start 116.15 102.55) (end 114.4 103.4) (width 0.5) (layer "F.Cu") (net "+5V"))
 (segment (start 114.4 103.4) (end 114.4 107) (width 0.5) (layer "F.Cu") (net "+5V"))
 (segment (start 118.3 99.3) (end 118.3 102.55) (width 0.5) (layer "F.Cu") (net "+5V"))
 (segment (start 118.3 102.55) (end 117.45 102.55) (width 0.5) (layer "F.Cu") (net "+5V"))
 (segment (start 114.4 107) (end 114.2 107.4) (width 0.5) (layer "F.Cu") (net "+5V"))
 (segment (start 116.6 94.8) (end 116 96) (width 0.5) (layer "F.Cu") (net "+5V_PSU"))
 (segment (start 117.3 91.5) (end 117.4 93) (width 0.5) (layer "F.Cu") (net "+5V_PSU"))
 (segment (start 116.7 90.45) (end 117.3 91.5) (width 0.5) (layer "F.Cu") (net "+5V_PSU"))
 (segment (start 116 96) (end 115.6 96.6) (width 0.5) (layer "F.Cu") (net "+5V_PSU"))
 (segment (start 115.6 96.6) (end 114.15 96.6) (width 0.5) (layer "F.Cu") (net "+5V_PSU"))
 (segment (start 107.75 109.1) (end 108.07 108.1) (width 0.25) (layer "F.Cu") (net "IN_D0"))
 (segment (start 104.6 108.1) (end 105 109.1) (width 0.25) (layer "F.Cu") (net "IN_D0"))
 (segment (start 105 109.1) (end 107.75 109.1) (width 0.25) (layer "F.Cu") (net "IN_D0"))
 (segment (start 104.6 108.1) (end 105.32 108.1) (width 0.25) (layer "F.Cu") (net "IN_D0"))
 (segment (start 101.5 91.3) (end 101.5 92.3) (width 0.25) (layer "F.Cu") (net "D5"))
 (segment (start 110.28 98.1) (end 111.1 98.1) (width 0.25) (layer "F.Cu") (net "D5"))
 (via (at 111.1 98.1) (size 0.6) (drill 0.3) (layers "F.Cu" "B.Cu") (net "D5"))
 (via (at 101.5 92.3) (size 0.6) (drill 0.3) (layers "F.Cu" "B.Cu") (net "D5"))
 (segment (start 101.5 97.15) (end 101.5 92.3) (width 0.25) (layer "B.Cu") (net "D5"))
 (segment (start 111.6 97.15) (end 101.5 97.15) (width 0.25) (layer "B.Cu") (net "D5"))
 (segment (start 111.6 98.1) (end 111.6 97.15) (width 0.25) (layer "B.Cu") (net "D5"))
 (segment (start 111.1 98.1) (end 111.6 98.1) (width 0.25) (layer "B.Cu") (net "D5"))
 (segment (start 83.4 108) (end 84.6 109.175) (width 0.8) (layer "F.Cu") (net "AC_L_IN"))
 (segment (start 84.6 109.175) (end 90.5 109.175) (width 0.8) (layer "F.Cu") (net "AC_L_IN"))
 (segment (start 89.5 100.65) (end 87.3 100.65) (width 0.8) (layer "F.Cu") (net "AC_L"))
 (segment (start 90.5 99.825) (end 90.8 93.35) (width 0.8) (layer "F.Cu") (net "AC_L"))
 (segment (start 90.5 99.825) (end 89.5 100.65) (width 0.8) (layer "F.Cu") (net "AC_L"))
 (segment (start 109.63 108.1) (end 111.3 108.4) (width 0.25) (layer "F.Cu") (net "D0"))
 (segment (start 114.2 94.4) (end 115.1 95) (width 0.25) (layer "F.Cu") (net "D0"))
 (via (at 111.3 108.4) (size 0.6) (drill 0.3) (layers "F.Cu" "B.Cu") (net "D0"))
 (via (at 115.1 95) (size 0.6) (drill 0.3) (layers "F.Cu" "B.Cu") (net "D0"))
 (segment (start 115.1 108.4) (end 115.1 95) (width 0.25) (layer "B.Cu") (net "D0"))
 (segment (start 111.3 108.4) (end 115.1 108.4) (width 0.25) (layer "B.Cu") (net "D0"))
 (segment (start 111.66 91.3) (end 111.66 92.3) (width 0.25) (layer "F.Cu") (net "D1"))
 (segment (start 109.63 106.1) (end 111.15 107.3) (width 0.25) (layer "F.Cu") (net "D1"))
 (via (at 111.66 92.3) (size 0.6) (drill 0.3) (layers "F.Cu" "B.Cu") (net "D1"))
 (via (at 111.15 107.3) (size 0.6) (drill 0.3) (layers "F.Cu" "B.Cu") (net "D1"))
 (segment (start 114.4 92.6) (end 111.66 92.6) (width 0.25) (layer "B.Cu") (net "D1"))
 (segment (start 111.66 92.6) (end 111.66 92.3) (width 0.25) (layer "B.Cu") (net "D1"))
 (segment (start 114.4 107.3) (end 114.4 92.6) (width 0.25) (layer "B.Cu") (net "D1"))
 (segment (start 111.15 107.3) (end 114.4 107.3) (width 0.25) (layer "B.Cu") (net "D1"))
 (segment (start 104.6 106.1) (end 105 105.1) (width 0.25) (layer "F.Cu") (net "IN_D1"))
 (segment (start 104.6 106.1) (end 105.32 106.1) (width 0.25) (layer "F.Cu") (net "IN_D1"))
 (segment (start 105 105.1) (end 107.75 105.1) (width 0.25) (layer "F.Cu") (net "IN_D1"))
 (segment (start 107.75 105.1) (end 108.07 106.1) (width 0.25) (layer "F.Cu") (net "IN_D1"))
 (segment (start 85 97.4) (end 87.3 95.65) (width 0.8) (layer "F.Cu") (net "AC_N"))
 (segment (start 83.4 97.4) (end 85 97.4) (width 0.8) (layer "F.Cu") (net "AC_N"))
 (segment (start 83.4 103) (end 83.4 93.35) (width 0.8) (layer "F.Cu") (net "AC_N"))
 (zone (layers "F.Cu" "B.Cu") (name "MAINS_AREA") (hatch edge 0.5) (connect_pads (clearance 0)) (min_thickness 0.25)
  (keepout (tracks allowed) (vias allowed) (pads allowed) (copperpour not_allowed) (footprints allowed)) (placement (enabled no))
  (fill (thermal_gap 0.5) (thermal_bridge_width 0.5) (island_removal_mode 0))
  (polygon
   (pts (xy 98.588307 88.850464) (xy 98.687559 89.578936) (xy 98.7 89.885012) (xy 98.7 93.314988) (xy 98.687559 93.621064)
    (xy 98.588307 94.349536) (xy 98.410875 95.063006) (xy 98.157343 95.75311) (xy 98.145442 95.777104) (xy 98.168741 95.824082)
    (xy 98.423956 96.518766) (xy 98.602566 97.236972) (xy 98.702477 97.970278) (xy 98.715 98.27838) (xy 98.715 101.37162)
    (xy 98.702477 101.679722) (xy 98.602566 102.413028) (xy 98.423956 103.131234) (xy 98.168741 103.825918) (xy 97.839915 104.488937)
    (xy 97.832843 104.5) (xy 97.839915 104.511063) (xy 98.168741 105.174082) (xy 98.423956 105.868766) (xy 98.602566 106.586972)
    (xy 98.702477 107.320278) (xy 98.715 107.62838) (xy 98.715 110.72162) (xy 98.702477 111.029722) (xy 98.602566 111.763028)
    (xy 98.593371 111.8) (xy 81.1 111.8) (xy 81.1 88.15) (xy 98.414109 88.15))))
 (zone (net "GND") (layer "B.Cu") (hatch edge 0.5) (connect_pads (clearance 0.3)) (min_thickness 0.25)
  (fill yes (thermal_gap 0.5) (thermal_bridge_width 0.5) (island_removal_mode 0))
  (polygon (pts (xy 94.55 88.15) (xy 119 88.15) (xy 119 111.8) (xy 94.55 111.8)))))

